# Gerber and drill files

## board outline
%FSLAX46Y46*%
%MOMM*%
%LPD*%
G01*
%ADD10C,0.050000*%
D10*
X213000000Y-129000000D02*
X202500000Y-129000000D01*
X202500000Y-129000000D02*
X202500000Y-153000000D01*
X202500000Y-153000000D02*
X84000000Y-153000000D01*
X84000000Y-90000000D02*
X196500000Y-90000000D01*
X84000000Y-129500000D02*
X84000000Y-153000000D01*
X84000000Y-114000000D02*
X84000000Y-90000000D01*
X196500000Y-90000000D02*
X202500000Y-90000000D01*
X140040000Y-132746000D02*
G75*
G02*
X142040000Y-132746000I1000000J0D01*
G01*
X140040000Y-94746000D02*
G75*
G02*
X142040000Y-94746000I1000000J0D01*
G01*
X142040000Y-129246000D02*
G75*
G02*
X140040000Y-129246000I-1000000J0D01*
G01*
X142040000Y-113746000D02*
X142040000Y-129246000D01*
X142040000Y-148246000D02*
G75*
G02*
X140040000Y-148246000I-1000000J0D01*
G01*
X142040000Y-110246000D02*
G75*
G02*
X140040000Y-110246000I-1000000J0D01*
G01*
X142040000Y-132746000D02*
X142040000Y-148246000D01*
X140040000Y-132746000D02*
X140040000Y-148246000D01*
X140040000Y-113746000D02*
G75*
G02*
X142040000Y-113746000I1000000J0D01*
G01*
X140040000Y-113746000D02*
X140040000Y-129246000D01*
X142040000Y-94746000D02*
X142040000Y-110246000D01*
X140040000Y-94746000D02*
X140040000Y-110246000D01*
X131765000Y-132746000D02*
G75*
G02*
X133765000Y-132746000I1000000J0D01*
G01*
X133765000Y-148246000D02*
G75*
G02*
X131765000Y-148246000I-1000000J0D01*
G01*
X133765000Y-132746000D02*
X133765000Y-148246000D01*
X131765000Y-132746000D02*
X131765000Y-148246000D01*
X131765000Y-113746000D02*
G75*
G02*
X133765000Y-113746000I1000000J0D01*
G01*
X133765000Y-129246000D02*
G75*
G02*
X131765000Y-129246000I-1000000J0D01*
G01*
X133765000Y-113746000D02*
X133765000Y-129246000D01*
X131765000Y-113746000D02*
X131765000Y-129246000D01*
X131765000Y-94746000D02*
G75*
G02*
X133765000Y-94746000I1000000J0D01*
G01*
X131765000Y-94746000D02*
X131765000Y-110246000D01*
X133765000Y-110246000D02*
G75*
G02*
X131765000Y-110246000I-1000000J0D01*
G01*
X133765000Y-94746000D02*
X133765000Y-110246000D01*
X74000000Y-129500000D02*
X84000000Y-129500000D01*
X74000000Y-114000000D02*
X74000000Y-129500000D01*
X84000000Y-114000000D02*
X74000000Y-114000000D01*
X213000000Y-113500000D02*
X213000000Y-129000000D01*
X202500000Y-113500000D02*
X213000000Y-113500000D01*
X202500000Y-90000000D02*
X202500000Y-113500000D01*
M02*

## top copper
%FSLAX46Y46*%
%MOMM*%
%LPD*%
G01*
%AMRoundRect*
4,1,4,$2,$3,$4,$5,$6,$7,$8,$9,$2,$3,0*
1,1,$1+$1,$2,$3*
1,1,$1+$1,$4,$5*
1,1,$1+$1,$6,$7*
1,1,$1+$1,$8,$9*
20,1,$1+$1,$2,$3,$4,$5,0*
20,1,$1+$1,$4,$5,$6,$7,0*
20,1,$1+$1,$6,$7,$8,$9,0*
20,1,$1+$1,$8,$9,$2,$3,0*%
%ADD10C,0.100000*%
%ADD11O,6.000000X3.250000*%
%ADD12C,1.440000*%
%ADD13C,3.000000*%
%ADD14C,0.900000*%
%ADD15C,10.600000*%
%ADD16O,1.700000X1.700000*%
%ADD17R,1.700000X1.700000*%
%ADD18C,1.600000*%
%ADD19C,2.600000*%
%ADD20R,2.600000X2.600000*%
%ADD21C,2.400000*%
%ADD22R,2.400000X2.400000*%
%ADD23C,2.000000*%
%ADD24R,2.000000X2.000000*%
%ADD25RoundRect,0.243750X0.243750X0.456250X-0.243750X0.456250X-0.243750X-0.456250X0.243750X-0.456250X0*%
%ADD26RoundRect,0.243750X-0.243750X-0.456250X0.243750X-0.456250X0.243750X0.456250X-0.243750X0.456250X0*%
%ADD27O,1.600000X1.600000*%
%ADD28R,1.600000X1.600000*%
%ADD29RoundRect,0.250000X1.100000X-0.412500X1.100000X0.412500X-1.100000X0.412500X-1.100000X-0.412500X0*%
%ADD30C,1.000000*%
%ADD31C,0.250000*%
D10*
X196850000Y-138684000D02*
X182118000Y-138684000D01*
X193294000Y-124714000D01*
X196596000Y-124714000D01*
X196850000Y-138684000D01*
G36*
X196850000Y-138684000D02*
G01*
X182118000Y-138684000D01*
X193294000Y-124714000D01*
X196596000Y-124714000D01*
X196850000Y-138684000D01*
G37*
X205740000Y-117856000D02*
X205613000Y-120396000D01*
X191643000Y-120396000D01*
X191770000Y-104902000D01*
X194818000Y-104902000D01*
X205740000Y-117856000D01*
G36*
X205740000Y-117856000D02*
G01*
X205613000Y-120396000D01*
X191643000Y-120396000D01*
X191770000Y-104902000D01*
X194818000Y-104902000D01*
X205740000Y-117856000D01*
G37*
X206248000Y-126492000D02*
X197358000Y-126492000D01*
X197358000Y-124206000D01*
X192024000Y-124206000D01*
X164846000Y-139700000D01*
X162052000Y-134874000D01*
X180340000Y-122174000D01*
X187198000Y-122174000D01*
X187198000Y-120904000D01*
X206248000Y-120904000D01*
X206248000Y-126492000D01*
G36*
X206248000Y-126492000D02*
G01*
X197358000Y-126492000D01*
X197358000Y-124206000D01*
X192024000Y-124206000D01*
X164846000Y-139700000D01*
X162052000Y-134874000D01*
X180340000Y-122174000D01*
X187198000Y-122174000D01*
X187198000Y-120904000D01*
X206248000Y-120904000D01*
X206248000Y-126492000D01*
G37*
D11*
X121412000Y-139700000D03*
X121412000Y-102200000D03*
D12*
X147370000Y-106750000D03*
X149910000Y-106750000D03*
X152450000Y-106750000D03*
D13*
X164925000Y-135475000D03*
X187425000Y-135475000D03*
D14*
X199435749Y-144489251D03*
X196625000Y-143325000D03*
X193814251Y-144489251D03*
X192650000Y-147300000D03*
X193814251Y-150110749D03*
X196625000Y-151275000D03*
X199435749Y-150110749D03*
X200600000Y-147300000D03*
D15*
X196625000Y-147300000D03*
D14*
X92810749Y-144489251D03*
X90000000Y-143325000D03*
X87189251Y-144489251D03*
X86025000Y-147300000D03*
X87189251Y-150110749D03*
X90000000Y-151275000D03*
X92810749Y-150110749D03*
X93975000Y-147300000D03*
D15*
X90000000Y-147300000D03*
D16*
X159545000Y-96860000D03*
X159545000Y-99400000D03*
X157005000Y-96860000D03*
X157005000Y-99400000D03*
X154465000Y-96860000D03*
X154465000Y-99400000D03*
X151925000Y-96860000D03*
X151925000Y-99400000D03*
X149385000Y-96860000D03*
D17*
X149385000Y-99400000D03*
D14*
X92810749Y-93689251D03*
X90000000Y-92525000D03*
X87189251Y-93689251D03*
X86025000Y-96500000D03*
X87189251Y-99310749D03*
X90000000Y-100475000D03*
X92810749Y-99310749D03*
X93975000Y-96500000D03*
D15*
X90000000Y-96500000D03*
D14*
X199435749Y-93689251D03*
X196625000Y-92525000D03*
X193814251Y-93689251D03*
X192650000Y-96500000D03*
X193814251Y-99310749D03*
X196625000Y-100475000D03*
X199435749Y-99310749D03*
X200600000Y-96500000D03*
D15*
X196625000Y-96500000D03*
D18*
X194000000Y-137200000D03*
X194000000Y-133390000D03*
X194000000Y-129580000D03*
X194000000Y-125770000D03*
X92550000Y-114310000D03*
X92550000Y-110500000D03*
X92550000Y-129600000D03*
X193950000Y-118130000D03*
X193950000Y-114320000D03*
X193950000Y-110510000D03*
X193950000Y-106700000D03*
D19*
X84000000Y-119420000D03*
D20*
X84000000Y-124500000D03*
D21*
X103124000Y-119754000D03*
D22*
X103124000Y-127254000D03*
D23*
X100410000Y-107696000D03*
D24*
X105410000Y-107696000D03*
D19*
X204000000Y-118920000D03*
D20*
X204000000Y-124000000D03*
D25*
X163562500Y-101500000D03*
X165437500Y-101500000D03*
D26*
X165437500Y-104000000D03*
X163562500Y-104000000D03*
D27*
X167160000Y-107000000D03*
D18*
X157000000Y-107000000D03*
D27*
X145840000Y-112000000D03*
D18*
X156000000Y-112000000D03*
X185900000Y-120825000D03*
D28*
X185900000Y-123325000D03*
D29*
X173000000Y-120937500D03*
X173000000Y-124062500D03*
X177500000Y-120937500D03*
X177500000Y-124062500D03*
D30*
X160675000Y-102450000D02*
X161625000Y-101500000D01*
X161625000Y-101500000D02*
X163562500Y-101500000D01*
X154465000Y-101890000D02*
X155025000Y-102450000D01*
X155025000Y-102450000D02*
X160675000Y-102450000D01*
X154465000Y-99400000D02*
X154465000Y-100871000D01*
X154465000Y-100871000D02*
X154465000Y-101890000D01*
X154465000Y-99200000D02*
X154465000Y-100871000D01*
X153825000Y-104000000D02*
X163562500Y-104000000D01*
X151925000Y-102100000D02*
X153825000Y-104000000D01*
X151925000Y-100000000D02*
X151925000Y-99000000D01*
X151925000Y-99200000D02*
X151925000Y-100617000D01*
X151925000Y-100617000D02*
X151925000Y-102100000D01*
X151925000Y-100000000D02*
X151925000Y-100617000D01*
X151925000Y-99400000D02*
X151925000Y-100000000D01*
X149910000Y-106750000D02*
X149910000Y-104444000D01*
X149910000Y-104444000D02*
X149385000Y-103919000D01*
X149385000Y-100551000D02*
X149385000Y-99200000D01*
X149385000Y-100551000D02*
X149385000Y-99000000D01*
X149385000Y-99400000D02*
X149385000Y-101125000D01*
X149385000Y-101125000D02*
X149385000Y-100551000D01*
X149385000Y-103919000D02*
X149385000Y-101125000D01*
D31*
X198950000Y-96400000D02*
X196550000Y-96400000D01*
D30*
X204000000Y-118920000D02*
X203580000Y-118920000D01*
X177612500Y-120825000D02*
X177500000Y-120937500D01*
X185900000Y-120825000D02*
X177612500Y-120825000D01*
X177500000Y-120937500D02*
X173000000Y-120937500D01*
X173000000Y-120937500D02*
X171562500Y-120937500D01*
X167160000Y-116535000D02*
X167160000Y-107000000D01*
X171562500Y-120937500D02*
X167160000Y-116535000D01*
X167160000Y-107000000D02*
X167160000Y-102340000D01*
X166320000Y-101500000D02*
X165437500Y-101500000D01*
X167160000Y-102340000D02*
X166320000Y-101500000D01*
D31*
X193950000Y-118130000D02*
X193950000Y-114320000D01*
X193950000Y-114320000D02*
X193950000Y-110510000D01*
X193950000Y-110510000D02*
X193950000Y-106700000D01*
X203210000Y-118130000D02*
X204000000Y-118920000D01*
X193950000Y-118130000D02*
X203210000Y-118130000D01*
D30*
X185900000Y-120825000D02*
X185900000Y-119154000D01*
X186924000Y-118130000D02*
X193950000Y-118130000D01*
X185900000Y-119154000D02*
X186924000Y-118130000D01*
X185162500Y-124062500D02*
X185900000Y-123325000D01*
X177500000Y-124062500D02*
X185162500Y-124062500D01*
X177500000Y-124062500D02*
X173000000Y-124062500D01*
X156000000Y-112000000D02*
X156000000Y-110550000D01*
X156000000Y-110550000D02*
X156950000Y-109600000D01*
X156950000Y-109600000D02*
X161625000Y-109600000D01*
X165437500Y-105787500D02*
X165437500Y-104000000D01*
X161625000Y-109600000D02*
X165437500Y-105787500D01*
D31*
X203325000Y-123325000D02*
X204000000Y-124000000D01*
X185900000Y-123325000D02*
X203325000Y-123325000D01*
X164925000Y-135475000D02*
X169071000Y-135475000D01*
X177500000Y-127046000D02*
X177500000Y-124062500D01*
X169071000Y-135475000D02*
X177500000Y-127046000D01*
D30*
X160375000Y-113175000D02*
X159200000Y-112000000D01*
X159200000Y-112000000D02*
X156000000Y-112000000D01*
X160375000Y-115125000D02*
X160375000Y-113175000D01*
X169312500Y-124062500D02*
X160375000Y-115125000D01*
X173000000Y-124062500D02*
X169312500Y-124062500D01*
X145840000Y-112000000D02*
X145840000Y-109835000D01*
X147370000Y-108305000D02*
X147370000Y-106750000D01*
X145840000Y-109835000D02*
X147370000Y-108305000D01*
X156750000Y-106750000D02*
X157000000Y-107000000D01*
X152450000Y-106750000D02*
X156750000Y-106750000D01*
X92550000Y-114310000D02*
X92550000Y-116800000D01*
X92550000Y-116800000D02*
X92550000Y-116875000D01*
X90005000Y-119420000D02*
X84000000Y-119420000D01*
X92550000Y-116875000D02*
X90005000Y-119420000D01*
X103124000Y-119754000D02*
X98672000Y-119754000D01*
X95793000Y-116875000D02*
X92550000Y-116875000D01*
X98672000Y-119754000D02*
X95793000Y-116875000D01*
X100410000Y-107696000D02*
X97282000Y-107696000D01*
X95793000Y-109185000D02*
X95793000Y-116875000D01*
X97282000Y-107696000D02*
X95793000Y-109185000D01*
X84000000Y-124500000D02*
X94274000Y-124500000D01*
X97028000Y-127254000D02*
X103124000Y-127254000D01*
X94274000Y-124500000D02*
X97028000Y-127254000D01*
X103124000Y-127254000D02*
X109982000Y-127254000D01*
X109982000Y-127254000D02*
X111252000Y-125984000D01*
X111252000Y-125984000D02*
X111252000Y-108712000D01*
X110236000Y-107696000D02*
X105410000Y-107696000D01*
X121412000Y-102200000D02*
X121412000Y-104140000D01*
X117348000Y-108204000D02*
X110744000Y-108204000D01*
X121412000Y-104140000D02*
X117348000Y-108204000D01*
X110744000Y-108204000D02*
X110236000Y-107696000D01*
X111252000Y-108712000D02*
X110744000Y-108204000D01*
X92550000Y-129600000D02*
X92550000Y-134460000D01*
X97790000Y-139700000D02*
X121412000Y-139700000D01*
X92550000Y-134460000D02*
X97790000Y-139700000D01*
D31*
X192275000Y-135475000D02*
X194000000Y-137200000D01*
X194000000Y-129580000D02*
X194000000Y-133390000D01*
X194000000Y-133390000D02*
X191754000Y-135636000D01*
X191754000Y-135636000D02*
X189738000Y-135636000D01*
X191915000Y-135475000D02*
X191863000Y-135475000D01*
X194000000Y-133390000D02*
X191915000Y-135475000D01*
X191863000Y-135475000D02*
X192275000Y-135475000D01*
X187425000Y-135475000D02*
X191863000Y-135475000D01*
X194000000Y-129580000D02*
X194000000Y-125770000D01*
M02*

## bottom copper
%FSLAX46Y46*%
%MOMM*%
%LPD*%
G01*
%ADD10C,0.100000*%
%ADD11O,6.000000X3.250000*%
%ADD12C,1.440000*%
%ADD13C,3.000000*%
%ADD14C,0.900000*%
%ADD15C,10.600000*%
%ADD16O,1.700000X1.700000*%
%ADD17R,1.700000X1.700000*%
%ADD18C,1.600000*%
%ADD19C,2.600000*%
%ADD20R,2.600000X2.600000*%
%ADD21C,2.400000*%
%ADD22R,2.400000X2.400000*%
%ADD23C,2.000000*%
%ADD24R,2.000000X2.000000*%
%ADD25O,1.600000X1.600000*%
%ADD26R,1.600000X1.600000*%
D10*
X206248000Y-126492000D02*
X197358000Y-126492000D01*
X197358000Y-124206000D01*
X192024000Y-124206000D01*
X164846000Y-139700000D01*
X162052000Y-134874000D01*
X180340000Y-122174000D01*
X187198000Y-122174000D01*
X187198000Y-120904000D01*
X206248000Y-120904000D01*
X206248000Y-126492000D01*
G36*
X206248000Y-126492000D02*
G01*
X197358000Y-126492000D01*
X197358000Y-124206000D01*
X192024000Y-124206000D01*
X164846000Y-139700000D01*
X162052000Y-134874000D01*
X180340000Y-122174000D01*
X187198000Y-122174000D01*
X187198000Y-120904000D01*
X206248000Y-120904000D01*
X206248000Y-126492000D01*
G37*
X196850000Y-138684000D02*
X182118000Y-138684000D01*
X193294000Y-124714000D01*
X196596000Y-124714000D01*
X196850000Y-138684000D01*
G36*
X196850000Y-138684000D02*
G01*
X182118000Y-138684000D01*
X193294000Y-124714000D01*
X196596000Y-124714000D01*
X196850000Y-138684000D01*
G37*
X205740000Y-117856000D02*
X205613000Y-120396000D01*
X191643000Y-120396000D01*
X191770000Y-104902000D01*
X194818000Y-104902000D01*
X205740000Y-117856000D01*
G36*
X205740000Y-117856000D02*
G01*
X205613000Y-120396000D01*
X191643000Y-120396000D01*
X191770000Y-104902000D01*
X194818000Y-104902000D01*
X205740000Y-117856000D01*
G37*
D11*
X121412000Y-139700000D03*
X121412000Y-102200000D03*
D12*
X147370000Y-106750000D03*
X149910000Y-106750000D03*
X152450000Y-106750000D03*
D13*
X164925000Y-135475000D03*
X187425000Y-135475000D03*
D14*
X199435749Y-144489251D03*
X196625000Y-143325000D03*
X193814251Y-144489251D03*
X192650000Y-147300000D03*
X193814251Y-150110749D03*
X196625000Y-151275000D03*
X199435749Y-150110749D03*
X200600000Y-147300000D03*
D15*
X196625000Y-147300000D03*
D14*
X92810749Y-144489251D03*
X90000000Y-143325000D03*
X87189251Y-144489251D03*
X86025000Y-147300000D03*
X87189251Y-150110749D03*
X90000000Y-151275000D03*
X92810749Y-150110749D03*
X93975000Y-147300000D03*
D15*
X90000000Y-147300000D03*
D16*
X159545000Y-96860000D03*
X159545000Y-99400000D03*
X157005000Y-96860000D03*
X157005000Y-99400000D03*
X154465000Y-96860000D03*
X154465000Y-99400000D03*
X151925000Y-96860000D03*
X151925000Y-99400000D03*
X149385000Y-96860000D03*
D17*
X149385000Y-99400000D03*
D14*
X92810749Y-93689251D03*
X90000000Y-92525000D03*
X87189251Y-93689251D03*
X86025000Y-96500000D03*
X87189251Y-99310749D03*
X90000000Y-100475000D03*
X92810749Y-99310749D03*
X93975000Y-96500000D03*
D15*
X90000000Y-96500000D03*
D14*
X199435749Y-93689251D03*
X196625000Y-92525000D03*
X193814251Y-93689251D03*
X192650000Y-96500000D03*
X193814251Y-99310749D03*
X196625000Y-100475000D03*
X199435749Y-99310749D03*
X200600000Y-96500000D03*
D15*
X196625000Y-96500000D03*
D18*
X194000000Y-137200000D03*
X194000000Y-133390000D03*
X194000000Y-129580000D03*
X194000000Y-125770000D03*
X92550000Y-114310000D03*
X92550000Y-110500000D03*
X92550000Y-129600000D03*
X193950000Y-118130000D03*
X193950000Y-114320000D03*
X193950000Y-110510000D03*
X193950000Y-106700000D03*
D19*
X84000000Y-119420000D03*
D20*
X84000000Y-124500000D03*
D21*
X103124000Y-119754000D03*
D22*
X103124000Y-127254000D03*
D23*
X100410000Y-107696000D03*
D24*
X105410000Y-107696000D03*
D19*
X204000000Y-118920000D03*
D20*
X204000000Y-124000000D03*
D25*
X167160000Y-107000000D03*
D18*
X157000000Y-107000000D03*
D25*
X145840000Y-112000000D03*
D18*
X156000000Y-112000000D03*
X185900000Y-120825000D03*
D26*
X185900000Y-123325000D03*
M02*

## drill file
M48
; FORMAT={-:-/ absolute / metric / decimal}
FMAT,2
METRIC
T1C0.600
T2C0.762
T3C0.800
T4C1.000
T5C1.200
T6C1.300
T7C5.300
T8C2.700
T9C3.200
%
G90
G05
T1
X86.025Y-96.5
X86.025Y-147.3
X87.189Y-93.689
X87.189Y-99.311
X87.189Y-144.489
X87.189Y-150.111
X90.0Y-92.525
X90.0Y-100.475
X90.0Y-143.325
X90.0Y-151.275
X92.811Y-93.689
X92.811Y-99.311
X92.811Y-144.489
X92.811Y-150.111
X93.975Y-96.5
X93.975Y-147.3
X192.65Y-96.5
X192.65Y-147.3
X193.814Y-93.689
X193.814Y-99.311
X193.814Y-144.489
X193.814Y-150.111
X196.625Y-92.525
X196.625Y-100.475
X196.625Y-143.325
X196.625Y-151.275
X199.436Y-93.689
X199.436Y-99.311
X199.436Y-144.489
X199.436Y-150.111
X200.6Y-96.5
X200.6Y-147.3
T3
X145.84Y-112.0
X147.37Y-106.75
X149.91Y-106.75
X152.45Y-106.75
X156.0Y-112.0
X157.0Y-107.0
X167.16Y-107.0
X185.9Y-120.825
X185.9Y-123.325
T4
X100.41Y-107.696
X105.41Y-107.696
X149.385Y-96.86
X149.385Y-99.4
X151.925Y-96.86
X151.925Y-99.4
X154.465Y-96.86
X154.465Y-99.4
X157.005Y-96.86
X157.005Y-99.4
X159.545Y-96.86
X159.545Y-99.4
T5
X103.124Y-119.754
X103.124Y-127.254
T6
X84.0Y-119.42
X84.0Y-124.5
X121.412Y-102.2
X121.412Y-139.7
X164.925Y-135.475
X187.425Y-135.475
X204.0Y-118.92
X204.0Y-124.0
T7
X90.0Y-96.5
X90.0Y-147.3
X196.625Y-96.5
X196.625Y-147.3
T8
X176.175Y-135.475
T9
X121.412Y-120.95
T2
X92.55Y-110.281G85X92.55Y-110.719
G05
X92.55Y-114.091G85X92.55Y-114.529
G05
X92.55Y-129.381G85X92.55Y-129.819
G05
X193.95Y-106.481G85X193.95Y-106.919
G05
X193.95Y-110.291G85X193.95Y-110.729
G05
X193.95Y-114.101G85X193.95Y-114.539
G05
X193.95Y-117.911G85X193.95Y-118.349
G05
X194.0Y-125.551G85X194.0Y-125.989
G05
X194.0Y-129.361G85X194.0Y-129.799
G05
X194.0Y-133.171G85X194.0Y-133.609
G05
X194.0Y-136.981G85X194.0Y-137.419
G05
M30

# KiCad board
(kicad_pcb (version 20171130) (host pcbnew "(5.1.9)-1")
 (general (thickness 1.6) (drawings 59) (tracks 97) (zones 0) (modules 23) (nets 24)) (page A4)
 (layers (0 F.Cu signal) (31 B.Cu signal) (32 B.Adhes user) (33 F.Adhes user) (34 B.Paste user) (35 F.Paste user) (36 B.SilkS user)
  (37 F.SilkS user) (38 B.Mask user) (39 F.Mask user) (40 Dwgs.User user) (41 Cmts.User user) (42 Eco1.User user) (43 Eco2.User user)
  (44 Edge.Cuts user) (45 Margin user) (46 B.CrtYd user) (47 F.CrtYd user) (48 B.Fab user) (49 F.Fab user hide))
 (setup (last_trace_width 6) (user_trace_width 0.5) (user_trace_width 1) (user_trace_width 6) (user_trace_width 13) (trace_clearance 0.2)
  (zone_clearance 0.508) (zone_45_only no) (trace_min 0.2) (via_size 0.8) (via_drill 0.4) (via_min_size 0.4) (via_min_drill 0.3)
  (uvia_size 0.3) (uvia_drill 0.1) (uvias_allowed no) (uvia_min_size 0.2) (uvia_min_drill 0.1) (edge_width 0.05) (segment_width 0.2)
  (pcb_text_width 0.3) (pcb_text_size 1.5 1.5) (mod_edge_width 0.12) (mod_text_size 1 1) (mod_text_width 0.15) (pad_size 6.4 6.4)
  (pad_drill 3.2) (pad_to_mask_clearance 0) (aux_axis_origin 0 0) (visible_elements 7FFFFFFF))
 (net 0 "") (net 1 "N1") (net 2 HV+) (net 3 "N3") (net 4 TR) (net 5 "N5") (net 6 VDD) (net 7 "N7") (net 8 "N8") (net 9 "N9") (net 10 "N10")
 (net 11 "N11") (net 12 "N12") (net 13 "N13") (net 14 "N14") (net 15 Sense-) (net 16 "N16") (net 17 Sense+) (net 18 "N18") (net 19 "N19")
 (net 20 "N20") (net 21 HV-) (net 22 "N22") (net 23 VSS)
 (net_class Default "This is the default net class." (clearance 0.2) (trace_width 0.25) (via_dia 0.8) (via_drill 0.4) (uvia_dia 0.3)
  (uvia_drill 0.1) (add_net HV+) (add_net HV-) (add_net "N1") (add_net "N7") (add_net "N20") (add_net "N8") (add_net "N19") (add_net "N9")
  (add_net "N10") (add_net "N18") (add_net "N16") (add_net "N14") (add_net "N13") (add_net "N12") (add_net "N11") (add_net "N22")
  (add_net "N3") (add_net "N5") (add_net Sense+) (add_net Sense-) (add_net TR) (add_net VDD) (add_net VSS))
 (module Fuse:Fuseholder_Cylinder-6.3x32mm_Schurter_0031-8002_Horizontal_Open (layer F.Cu) (at 121.412 139.7 90)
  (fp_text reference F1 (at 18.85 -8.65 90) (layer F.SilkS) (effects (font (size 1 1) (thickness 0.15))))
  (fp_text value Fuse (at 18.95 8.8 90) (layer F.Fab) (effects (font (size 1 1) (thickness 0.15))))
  (pad 1 thru_hole oval (at 0 0 90) (size 3.25 6) (drill 1.3) (layers *.Cu *.Mask) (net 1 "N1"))
  (pad 2 thru_hole oval (at 37.5 0 90) (size 3.25 6) (drill 1.3) (layers *.Cu *.Mask) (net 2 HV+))
  (pad "" np_thru_hole circle (at 18.75 0 90) (size 3.2 3.2) (drill 3.2) (layers *.Cu *.Mask)))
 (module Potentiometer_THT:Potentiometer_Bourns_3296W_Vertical (layer F.Cu) (at 152.45 106.75)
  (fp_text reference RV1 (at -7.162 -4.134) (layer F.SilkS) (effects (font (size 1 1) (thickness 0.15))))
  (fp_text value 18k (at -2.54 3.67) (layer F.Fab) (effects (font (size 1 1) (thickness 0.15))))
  (pad 3 thru_hole circle (at -5.08 0) (size 1.44 1.44) (drill 0.8) (layers *.Cu *.Mask) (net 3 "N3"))
  (pad 2 thru_hole circle (at -2.54 0) (size 1.44 1.44) (drill 0.8) (layers *.Cu *.Mask) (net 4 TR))
  (pad 1 thru_hole circle (at 0 0) (size 1.44 1.44) (drill 0.8) (layers *.Cu *.Mask) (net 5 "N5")))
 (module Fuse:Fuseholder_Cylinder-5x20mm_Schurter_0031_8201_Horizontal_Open (layer F.Cu) (at 187.425 135.475 180)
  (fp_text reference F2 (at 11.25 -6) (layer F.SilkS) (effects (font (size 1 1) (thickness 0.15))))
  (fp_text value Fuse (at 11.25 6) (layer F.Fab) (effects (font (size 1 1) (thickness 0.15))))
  (pad "" np_thru_hole circle (at 11.25 0 180) (size 2.7 2.7) (drill 2.7) (layers *.Cu *.Mask))
  (pad 2 thru_hole circle (at 22.5 0 180) (size 3 3) (drill 1.3) (layers *.Cu *.Mask) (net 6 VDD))
  (pad 1 thru_hole circle (at 0 0 180) (size 3 3) (drill 1.3) (layers *.Cu *.Mask) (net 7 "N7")))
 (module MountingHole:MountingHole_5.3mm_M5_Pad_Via (layer F.Cu) (at 196.625 147.3)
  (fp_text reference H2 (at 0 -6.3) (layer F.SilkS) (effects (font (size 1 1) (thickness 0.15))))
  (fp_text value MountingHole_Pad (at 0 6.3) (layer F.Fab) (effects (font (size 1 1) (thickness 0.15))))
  (pad 1 thru_hole circle (at 2.810749 -2.810749) (size 0.9 0.9) (drill 0.6) (layers *.Cu *.Mask) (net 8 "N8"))
  (pad 1 thru_hole circle (at 0 -3.975) (size 0.9 0.9) (drill 0.6) (layers *.Cu *.Mask) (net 8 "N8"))
  (pad 1 thru_hole circle (at -2.810749 -2.810749) (size 0.9 0.9) (drill 0.6) (layers *.Cu *.Mask) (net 8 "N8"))
  (pad 1 thru_hole circle (at -3.975 0) (size 0.9 0.9) (drill 0.6) (layers *.Cu *.Mask) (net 8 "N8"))
  (pad 1 thru_hole circle (at -2.810749 2.810749) (size 0.9 0.9) (drill 0.6) (layers *.Cu *.Mask) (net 8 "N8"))
  (pad 1 thru_hole circle (at 0 3.975) (size 0.9 0.9) (drill 0.6) (layers *.Cu *.Mask) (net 8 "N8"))
  (pad 1 thru_hole circle (at 2.810749 2.810749) (size 0.9 0.9) (drill 0.6) (layers *.Cu *.Mask) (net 8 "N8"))
  (pad 1 thru_hole circle (at 3.975 0) (size 0.9 0.9) (drill 0.6) (layers *.Cu *.Mask) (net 8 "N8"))
  (pad 1 thru_hole circle (at 0 0) (size 10.6 10.6) (drill 5.3) (layers *.Cu *.Mask) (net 8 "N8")))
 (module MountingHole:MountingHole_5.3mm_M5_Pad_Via (layer F.Cu) (at 90 147.3)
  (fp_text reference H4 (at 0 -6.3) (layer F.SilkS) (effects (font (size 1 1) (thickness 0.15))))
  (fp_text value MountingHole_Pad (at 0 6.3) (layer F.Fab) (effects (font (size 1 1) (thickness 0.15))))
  (pad 1 thru_hole circle (at 2.810749 -2.810749) (size 0.9 0.9) (drill 0.6) (layers *.Cu *.Mask) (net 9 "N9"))
  (pad 1 thru_hole circle (at 0 -3.975) (size 0.9 0.9) (drill 0.6) (layers *.Cu *.Mask) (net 9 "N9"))
  (pad 1 thru_hole circle (at -2.810749 -2.810749) (size 0.9 0.9) (drill 0.6) (layers *.Cu *.Mask) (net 9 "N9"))
  (pad 1 thru_hole circle (at -3.975 0) (size 0.9 0.9) (drill 0.6) (layers *.Cu *.Mask) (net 9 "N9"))
  (pad 1 thru_hole circle (at -2.810749 2.810749) (size 0.9 0.9) (drill 0.6) (layers *.Cu *.Mask) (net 9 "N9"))
  (pad 1 thru_hole circle (at 0 3.975) (size 0.9 0.9) (drill 0.6) (layers *.Cu *.Mask) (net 9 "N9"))
  (pad 1 thru_hole circle (at 2.810749 2.810749) (size 0.9 0.9) (drill 0.6) (layers *.Cu *.Mask) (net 9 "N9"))
  (pad 1 thru_hole circle (at 3.975 0) (size 0.9 0.9) (drill 0.6) (layers *.Cu *.Mask) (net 9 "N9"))
  (pad 1 thru_hole circle (at 0 0) (size 10.6 10.6) (drill 5.3) (layers *.Cu *.Mask) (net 9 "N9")))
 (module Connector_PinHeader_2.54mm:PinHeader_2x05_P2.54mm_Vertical (layer F.Cu) (at 149.385 99.4 90)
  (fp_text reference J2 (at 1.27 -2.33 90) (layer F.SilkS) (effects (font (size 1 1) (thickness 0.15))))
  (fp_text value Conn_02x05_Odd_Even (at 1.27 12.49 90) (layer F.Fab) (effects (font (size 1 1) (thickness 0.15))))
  (pad 10 thru_hole oval (at 2.54 10.16 90) (size 1.7 1.7) (drill 1) (layers *.Cu *.Mask) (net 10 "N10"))
  (pad 9 thru_hole oval (at 0 10.16 90) (size 1.7 1.7) (drill 1) (layers *.Cu *.Mask) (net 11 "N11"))
  (pad 8 thru_hole oval (at 2.54 7.62 90) (size 1.7 1.7) (drill 1) (layers *.Cu *.Mask) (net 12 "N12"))
  (pad 7 thru_hole oval (at 0 7.62 90) (size 1.7 1.7) (drill 1) (layers *.Cu *.Mask) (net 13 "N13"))
  (pad 6 thru_hole oval (at 2.54 5.08 90) (size 1.7 1.7) (drill 1) (layers *.Cu *.Mask) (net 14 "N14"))
  (pad 5 thru_hole oval (at 0 5.08 90) (size 1.7 1.7) (drill 1) (layers *.Cu *.Mask) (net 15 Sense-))
  (pad 4 thru_hole oval (at 2.54 2.54 90) (size 1.7 1.7) (drill 1) (layers *.Cu *.Mask) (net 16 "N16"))
  (pad 3 thru_hole oval (at 0 2.54 90) (size 1.7 1.7) (drill 1) (layers *.Cu *.Mask) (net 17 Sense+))
  (pad 2 thru_hole oval (at 2.54 0 90) (size 1.7 1.7) (drill 1) (layers *.Cu *.Mask) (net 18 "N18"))
  (pad 1 thru_hole rect (at 0 0 90) (size 1.7 1.7) (drill 1) (layers *.Cu *.Mask) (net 4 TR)))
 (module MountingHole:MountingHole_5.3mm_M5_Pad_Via (layer F.Cu) (at 90 96.5)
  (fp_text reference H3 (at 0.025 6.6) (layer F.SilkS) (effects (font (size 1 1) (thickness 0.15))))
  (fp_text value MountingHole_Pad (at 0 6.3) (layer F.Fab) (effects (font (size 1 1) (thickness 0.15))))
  (pad 1 thru_hole circle (at 2.810749 -2.810749) (size 0.9 0.9) (drill 0.6) (layers *.Cu *.Mask) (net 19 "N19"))
  (pad 1 thru_hole circle (at 0 -3.975) (size 0.9 0.9) (drill 0.6) (layers *.Cu *.Mask) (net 19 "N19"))
  (pad 1 thru_hole circle (at -2.810749 -2.810749) (size 0.9 0.9) (drill 0.6) (layers *.Cu *.Mask) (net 19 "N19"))
  (pad 1 thru_hole circle (at -3.975 0) (size 0.9 0.9) (drill 0.6) (layers *.Cu *.Mask) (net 19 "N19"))
  (pad 1 thru_hole circle (at -2.810749 2.810749) (size 0.9 0.9) (drill 0.6) (layers *.Cu *.Mask) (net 19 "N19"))
  (pad 1 thru_hole circle (at 0 3.975) (size 0.9 0.9) (drill 0.6) (layers *.Cu *.Mask) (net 19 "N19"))
  (pad 1 thru_hole circle (at 2.810749 2.810749) (size 0.9 0.9) (drill 0.6) (layers *.Cu *.Mask) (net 19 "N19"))
  (pad 1 thru_hole circle (at 3.975 0) (size 0.9 0.9) (drill 0.6) (layers *.Cu *.Mask) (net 19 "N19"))
  (pad 1 thru_hole circle (at 0 0) (size 10.6 10.6) (drill 5.3) (layers *.Cu *.Mask) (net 19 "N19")))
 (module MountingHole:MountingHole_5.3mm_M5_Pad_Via (layer F.Cu) (at 196.625 96.5)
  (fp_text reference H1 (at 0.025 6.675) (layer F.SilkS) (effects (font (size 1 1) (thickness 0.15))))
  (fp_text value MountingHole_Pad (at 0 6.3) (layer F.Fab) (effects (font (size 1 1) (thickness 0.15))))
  (pad 1 thru_hole circle (at 2.810749 -2.810749) (size 0.9 0.9) (drill 0.6) (layers *.Cu *.Mask) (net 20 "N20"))
  (pad 1 thru_hole circle (at 0 -3.975) (size 0.9 0.9) (drill 0.6) (layers *.Cu *.Mask) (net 20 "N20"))
  (pad 1 thru_hole circle (at -2.810749 -2.810749) (size 0.9 0.9) (drill 0.6) (layers *.Cu *.Mask) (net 20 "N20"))
  (pad 1 thru_hole circle (at -3.975 0) (size 0.9 0.9) (drill 0.6) (layers *.Cu *.Mask) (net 20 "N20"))
  (pad 1 thru_hole circle (at -2.810749 2.810749) (size 0.9 0.9) (drill 0.6) (layers *.Cu *.Mask) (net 20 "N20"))
  (pad 1 thru_hole circle (at 0 3.975) (size 0.9 0.9) (drill 0.6) (layers *.Cu *.Mask) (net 20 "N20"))
  (pad 1 thru_hole circle (at 2.810749 2.810749) (size 0.9 0.9) (drill 0.6) (layers *.Cu *.Mask) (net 20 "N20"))
  (pad 1 thru_hole circle (at 3.975 0) (size 0.9 0.9) (drill 0.6) (layers *.Cu *.Mask) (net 20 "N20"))
  (pad 1 thru_hole circle (at 0 0) (size 10.6 10.6) (drill 5.3) (layers *.Cu *.Mask) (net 20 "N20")))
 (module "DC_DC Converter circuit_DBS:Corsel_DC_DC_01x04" (layer F.Cu) (at 194 130.85)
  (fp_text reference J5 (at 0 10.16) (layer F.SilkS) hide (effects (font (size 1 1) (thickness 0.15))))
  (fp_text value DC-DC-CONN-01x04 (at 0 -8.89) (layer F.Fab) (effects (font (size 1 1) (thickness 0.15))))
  (pad 4 thru_hole circle (at 0 6.35) (size 1.6 1.6) (drill oval 0.762 1.2) (layers *.Cu *.Mask) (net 7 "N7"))
  (pad 3 thru_hole circle (at 0 2.54) (size 1.6 1.6) (drill oval 0.762 1.2) (layers *.Cu *.Mask) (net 7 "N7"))
  (pad 2 thru_hole circle (at 0 -1.27) (size 1.6 1.6) (drill oval 0.762 1.2) (layers *.Cu *.Mask) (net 7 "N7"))
  (pad 1 thru_hole circle (at 0 -5.08) (size 1.6 1.6) (drill oval 0.762 1.2) (layers *.Cu *.Mask) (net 7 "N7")))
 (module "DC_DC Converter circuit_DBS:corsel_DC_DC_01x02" (layer F.Cu) (at 92.55 111.5)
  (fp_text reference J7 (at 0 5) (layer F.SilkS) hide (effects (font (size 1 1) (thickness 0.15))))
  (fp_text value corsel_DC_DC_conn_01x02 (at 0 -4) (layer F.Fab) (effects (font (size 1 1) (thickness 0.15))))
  (pad 2 thru_hole circle (at 0 2.81) (size 1.6 1.6) (drill oval 0.762 1.2) (layers *.Cu *.Mask) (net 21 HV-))
  (pad 1 thru_hole circle (at 0 -1) (size 1.6 1.6) (drill oval 0.762 1.2) (layers *.Cu *.Mask) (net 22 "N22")))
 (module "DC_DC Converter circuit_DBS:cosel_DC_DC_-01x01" (layer F.Cu) (at 92.55 129.6)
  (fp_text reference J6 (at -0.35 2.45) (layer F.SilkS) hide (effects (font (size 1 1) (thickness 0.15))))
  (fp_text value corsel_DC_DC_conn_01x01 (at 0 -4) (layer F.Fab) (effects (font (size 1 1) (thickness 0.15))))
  (pad 1 thru_hole circle (at 0 0) (size 1.6 1.6) (drill oval 0.762 1.2) (layers *.Cu *.Mask) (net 1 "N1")))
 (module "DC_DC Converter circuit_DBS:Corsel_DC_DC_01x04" (layer F.Cu) (at 193.95 111.78)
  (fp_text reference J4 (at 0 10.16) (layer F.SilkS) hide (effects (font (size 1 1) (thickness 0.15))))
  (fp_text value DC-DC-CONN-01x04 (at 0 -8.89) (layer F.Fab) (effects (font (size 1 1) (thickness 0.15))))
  (pad 4 thru_hole circle (at 0 6.35) (size 1.6 1.6) (drill oval 0.762 1.2) (layers *.Cu *.Mask) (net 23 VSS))
  (pad 3 thru_hole circle (at 0 2.54) (size 1.6 1.6) (drill oval 0.762 1.2) (layers *.Cu *.Mask) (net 23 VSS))
  (pad 2 thru_hole circle (at 0 -1.27) (size 1.6 1.6) (drill oval 0.762 1.2) (layers *.Cu *.Mask) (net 23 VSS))
  (pad 1 thru_hole circle (at 0 -5.08) (size 1.6 1.6) (drill oval 0.762 1.2) (layers *.Cu *.Mask) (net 23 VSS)))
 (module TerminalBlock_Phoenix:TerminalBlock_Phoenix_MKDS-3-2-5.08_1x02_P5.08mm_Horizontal (layer F.Cu) (at 84 124.5 90)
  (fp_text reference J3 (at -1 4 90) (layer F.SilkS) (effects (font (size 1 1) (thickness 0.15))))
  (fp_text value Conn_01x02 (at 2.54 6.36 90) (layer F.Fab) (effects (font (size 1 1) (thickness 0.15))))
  (pad 2 thru_hole circle (at 5.08 0 90) (size 2.6 2.6) (drill 1.3) (layers *.Cu *.Mask) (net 21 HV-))
  (pad 1 thru_hole rect (at 0 0 90) (size 2.6 2.6) (drill 1.3) (layers *.Cu *.Mask) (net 2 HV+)))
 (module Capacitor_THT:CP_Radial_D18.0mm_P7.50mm (layer F.Cu) (at 103.124 127.254 90)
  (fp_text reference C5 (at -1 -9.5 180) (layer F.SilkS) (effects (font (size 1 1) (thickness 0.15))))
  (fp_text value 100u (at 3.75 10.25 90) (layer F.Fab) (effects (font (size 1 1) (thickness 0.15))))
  (pad 2 thru_hole circle (at 7.5 0 90) (size 2.4 2.4) (drill 1.2) (layers *.Cu *.Mask) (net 21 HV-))
  (pad 1 thru_hole rect (at 0 0 90) (size 2.4 2.4) (drill 1.2) (layers *.Cu *.Mask) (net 2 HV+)))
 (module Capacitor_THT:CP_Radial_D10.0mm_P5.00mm (layer F.Cu) (at 105.41 107.696 180)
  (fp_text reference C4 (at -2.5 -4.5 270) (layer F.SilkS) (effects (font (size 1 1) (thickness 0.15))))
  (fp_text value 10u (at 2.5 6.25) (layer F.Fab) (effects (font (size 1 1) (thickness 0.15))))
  (pad 2 thru_hole circle (at 5 0 180) (size 2 2) (drill 1) (layers *.Cu *.Mask) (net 21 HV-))
  (pad 1 thru_hole rect (at 0 0 180) (size 2 2) (drill 1) (layers *.Cu *.Mask) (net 2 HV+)))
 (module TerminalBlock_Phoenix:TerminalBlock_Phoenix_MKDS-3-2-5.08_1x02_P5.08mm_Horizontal (layer F.Cu) (at 204 124 90)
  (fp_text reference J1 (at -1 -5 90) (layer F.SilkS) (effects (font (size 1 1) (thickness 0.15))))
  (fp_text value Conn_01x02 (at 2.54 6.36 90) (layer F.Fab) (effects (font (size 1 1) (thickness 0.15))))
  (pad 2 thru_hole circle (at 5.08 0 90) (size 2.6 2.6) (drill 1.3) (layers *.Cu *.Mask) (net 23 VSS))
  (pad 1 thru_hole rect (at 0 0 90) (size 2.6 2.6) (drill 1.3) (layers *.Cu *.Mask) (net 6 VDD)))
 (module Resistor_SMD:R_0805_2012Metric (layer F.Cu) (at 164.5 101.5 180)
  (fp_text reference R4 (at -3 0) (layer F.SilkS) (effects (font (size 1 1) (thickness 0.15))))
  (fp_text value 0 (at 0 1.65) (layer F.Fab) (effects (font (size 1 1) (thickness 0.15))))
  (pad 2 smd roundrect (at 0.9375 0 180) (size 0.975 1.4) (layers F.Cu F.Paste F.Mask) (roundrect_rratio 0.25) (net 15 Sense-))
  (pad 1 smd roundrect (at -0.9375 0 180) (size 0.975 1.4) (layers F.Cu F.Paste F.Mask) (roundrect_rratio 0.25) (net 23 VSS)))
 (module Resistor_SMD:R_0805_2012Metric (layer F.Cu) (at 164.5 104)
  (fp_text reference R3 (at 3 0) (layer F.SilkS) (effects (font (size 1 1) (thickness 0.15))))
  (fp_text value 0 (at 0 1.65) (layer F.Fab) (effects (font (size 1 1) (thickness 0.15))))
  (pad 2 smd roundrect (at 0.9375 0) (size 0.975 1.4) (layers F.Cu F.Paste F.Mask) (roundrect_rratio 0.25) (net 6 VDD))
  (pad 1 smd roundrect (at -0.9375 0) (size 0.975 1.4) (layers F.Cu F.Paste F.Mask) (roundrect_rratio 0.25) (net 17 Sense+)))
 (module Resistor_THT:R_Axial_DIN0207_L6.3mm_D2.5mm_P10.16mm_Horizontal (layer F.Cu) (at 157 107)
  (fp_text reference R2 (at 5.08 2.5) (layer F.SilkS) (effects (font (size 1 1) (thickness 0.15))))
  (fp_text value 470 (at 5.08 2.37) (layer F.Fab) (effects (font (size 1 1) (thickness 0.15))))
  (pad 2 thru_hole oval (at 10.16 0) (size 1.6 1.6) (drill 0.8) (layers *.Cu *.Mask) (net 23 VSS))
  (pad 1 thru_hole circle (at 0 0) (size 1.6 1.6) (drill 0.8) (layers *.Cu *.Mask) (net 5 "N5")))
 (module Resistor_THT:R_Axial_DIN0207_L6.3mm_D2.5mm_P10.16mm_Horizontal (layer F.Cu) (at 156 112 180)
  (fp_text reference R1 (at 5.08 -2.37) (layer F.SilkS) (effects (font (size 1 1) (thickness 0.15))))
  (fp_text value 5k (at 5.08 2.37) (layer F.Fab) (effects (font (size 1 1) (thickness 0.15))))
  (pad 2 thru_hole oval (at 10.16 0 180) (size 1.6 1.6) (drill 0.8) (layers *.Cu *.Mask) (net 3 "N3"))
  (pad 1 thru_hole circle (at 0 0 180) (size 1.6 1.6) (drill 0.8) (layers *.Cu *.Mask) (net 6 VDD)))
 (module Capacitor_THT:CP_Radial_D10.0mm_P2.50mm (layer F.Cu) (at 185.9 123.325 90)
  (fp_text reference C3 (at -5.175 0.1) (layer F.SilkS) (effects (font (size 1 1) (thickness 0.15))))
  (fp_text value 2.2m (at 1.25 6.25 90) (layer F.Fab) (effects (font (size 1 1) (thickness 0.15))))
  (pad 2 thru_hole circle (at 2.5 0 90) (size 1.6 1.6) (drill 0.8) (layers *.Cu *.Mask) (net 23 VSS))
  (pad 1 thru_hole rect (at 0 0 90) (size 1.6 1.6) (drill 0.8) (layers *.Cu *.Mask) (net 6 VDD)))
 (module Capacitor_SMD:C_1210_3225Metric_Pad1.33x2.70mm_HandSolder (layer F.Cu) (at 173 122.5 90)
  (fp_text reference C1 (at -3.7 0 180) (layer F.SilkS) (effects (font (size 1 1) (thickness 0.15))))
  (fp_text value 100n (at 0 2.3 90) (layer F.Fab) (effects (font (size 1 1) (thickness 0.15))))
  (pad 2 smd roundrect (at 1.5625 0 90) (size 1.325 2.7) (layers F.Cu F.Paste F.Mask) (roundrect_rratio 0.188679) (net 23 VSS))
  (pad 1 smd roundrect (at -1.5625 0 90) (size 1.325 2.7) (layers F.Cu F.Paste F.Mask) (roundrect_rratio 0.188679) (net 6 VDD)))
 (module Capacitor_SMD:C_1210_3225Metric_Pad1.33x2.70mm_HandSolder (layer F.Cu) (at 177.5 122.5 90)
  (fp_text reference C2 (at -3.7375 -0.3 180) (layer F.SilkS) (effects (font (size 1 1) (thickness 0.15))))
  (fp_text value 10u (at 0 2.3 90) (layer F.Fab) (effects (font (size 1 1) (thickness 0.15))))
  (pad 2 smd roundrect (at 1.5625 0 90) (size 1.325 2.7) (layers F.Cu F.Paste F.Mask) (roundrect_rratio 0.188679) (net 23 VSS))
  (pad 1 smd roundrect (at -1.5625 0 90) (size 1.325 2.7) (layers F.Cu F.Paste F.Mask) (roundrect_rratio 0.188679) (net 6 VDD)))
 (gr_poly (pts (xy 196.85 138.684) (xy 182.118 138.684) (xy 193.294 124.714) (xy 196.596 124.714)) (layer F.Cu) (width 0.1))
 (gr_poly
  (pts (xy 205.74 117.856) (xy 205.613 120.396) (xy 191.643 120.396) (xy 191.77 104.902) (xy 194.818 104.902)) (layer F.Cu) (width 0.1))
 (gr_poly
  (pts (xy 206.248 126.492) (xy 197.358 126.492) (xy 197.358 124.206) (xy 192.024 124.206) (xy 164.846 139.7) (xy 162.052 134.874)
   (xy 180.34 122.174) (xy 187.198 122.174) (xy 187.198 120.904) (xy 206.248 120.904))
  (layer F.Cu) (width 0.1))
 (gr_poly
  (pts (xy 206.248 126.492) (xy 197.358 126.492) (xy 197.358 124.206) (xy 192.024 124.206) (xy 164.846 139.7) (xy 162.052 134.874)
   (xy 180.34 122.174) (xy 187.198 122.174) (xy 187.198 120.904) (xy 206.248 120.904))
  (layer B.Cu) (width 0.1))
 (gr_poly (pts (xy 196.85 138.684) (xy 182.118 138.684) (xy 193.294 124.714) (xy 196.596 124.714)) (layer B.Cu) (width 0.1))
 (gr_poly
  (pts (xy 205.74 117.856) (xy 205.613 120.396) (xy 191.643 120.396) (xy 191.77 104.902) (xy 194.818 104.902)) (layer B.Cu) (width 0.1))
 (gr_line (start 213 129) (end 202.5 129) (layer Edge.Cuts) (width 0.05))
 (gr_line (start 202.5 129) (end 202.5 153) (layer Edge.Cuts) (width 0.05))
 (gr_line (start 202.5 153) (end 84 153) (layer Edge.Cuts) (width 0.05))
 (gr_line (start 84 90) (end 196.5 90) (layer Edge.Cuts) (width 0.05))
 (gr_line (start 84 129.5) (end 84 153) (layer Edge.Cuts) (width 0.05))
 (gr_line (start 84 114) (end 84 90) (layer Edge.Cuts) (width 0.05))
 (gr_line (start 196.5 90) (end 202.5 90) (layer Edge.Cuts) (width 0.05))
 (gr_arc (start 141.04 132.746) (end 142.04 132.746) (angle -180) (layer Edge.Cuts) (width 0.05))
 (gr_arc (start 141.04 94.746) (end 142.04 94.746) (angle -180) (layer Edge.Cuts) (width 0.05))
 (gr_arc (start 141.04 129.246) (end 140.04 129.246) (angle -180) (layer Edge.Cuts) (width 0.05))
 (gr_line (start 142.04 113.746) (end 142.04 129.246) (layer Edge.Cuts) (width 0.05))
 (gr_arc (start 141.04 148.246) (end 140.04 148.246) (angle -180) (layer Edge.Cuts) (width 0.05))
 (gr_arc (start 141.04 110.246) (end 140.04 110.246) (angle -180) (layer Edge.Cuts) (width 0.05))
 (gr_line (start 142.04 132.746) (end 142.04 148.246) (layer Edge.Cuts) (width 0.05))
 (gr_line (start 140.04 132.746) (end 140.04 148.246) (layer Edge.Cuts) (width 0.05))
 (gr_arc (start 141.04 113.746) (end 142.04 113.746) (angle -180) (layer Edge.Cuts) (width 0.05))
 (gr_line (start 140.04 113.746) (end 140.04 129.246) (layer Edge.Cuts) (width 0.05))
 (gr_line (start 142.04 94.746) (end 142.04 110.246) (layer Edge.Cuts) (width 0.05))
 (gr_line (start 140.04 94.746) (end 140.04 110.246) (layer Edge.Cuts) (width 0.05))
 (gr_arc (start 132.765 132.746) (end 133.765 132.746) (angle -180) (layer Edge.Cuts) (width 0.05))
 (gr_arc (start 132.765 148.246) (end 131.765 148.246) (angle -180) (layer Edge.Cuts) (width 0.05))
 (gr_line (start 133.765 132.746) (end 133.765 148.246) (layer Edge.Cuts) (width 0.05))
 (gr_line (start 131.765 132.746) (end 131.765 148.246) (layer Edge.Cuts) (width 0.05))
 (gr_arc (start 132.765 113.746) (end 133.765 113.746) (angle -180) (layer Edge.Cuts) (width 0.05))
 (gr_arc (start 132.765 129.246) (end 131.765 129.246) (angle -180) (layer Edge.Cuts) (width 0.05))
 (gr_line (start 133.765 113.746) (end 133.765 129.246) (layer Edge.Cuts) (width 0.05))
 (gr_line (start 131.765 113.746) (end 131.765 129.246) (layer Edge.Cuts) (width 0.05))
 (gr_arc (start 132.765 94.746) (end 133.765 94.746) (angle -180) (layer Edge.Cuts) (width 0.05))
 (gr_line (start 131.765 94.746) (end 131.765 110.246) (layer Edge.Cuts) (width 0.05))
 (gr_arc (start 132.765 110.246) (end 131.765 110.246) (angle -180) (layer Edge.Cuts) (width 0.05))
 (gr_line (start 133.765 94.746) (end 133.765 110.246) (layer Edge.Cuts) (width 0.05))
 (gr_line (start 74 129.5) (end 84 129.5) (layer Edge.Cuts) (width 0.05))
 (gr_line (start 74 114) (end 74 129.5) (layer Edge.Cuts) (width 0.05))
 (gr_line (start 84 114) (end 74 114) (layer Edge.Cuts) (width 0.05))
 (gr_line (start 213 113.5) (end 213 129) (layer Edge.Cuts) (width 0.05))
 (gr_line (start 202.5 113.5) (end 213 113.5) (layer Edge.Cuts) (width 0.05))
 (gr_line (start 202.5 90) (end 202.5 113.5) (layer Edge.Cuts) (width 0.05))
 (segment (start 160.675 102.45) (end 161.625 101.5) (width 1) (layer F.Cu) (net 15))
 (segment (start 161.625 101.5) (end 163.5625 101.5) (width 1) (layer F.Cu) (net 15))
 (segment (start 154.465 101.89) (end 155.025 102.45) (width 1) (layer F.Cu) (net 15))
 (segment (start 155.025 102.45) (end 160.675 102.45) (width 1) (layer F.Cu) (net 15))
 (segment (start 154.465 99.4) (end 154.465 100.871) (width 1) (layer F.Cu) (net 15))
 (segment (start 154.465 100.871) (end 154.465 101.89) (width 1) (layer F.Cu) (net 15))
 (segment (start 154.465 99.2) (end 154.465 100.871) (width 1) (layer F.Cu) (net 15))
 (segment (start 153.825 104) (end 163.5625 104) (width 1) (layer F.Cu) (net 17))
 (segment (start 151.925 102.1) (end 153.825 104) (width 1) (layer F.Cu) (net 17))
 (segment (start 151.925 100) (end 151.925 99) (width 1) (layer F.Cu) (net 17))
 (segment (start 151.925 99.2) (end 151.925 100.617) (width 1) (layer F.Cu) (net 17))
 (segment (start 151.925 100.617) (end 151.925 102.1) (width 1) (layer F.Cu) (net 17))
 (segment (start 151.925 100) (end 151.925 100.617) (width 1) (layer F.Cu) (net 17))
 (segment (start 151.925 99.4) (end 151.925 100) (width 1) (layer F.Cu) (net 17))
 (segment (start 149.91 106.75) (end 149.91 104.444) (width 1) (layer F.Cu) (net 4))
 (segment (start 149.91 104.444) (end 149.385 103.919) (width 1) (layer F.Cu) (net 4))
 (segment (start 149.385 100.551) (end 149.385 99.2) (width 1) (layer F.Cu) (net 4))
 (segment (start 149.385 100.551) (end 149.385 99) (width 1) (layer F.Cu) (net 4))
 (segment (start 149.385 99.4) (end 149.385 101.125) (width 1) (layer F.Cu) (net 4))
 (segment (start 149.385 101.125) (end 149.385 100.551) (width 1) (layer F.Cu) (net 4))
 (segment (start 149.385 103.919) (end 149.385 101.125) (width 1) (layer F.Cu) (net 4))
 (segment (start 198.95 96.4) (end 196.55 96.4) (width 0.25) (layer F.Cu) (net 20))
 (segment (start 204 118.92) (end 203.58 118.92) (width 1) (layer F.Cu) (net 23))
 (segment (start 177.6125 120.825) (end 177.5 120.9375) (width 1) (layer F.Cu) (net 23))
 (segment (start 185.9 120.825) (end 177.6125 120.825) (width 1) (layer F.Cu) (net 23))
 (segment (start 177.5 120.9375) (end 173 120.9375) (width 1) (layer F.Cu) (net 23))
 (segment (start 173 120.9375) (end 171.5625 120.9375) (width 1) (layer F.Cu) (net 23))
 (segment (start 167.16 116.535) (end 167.16 107) (width 1) (layer F.Cu) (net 23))
 (segment (start 171.5625 120.9375) (end 167.16 116.535) (width 1) (layer F.Cu) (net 23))
 (segment (start 167.16 107) (end 167.16 102.34) (width 1) (layer F.Cu) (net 23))
 (segment (start 166.32 101.5) (end 165.4375 101.5) (width 1) (layer F.Cu) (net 23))
 (segment (start 167.16 102.34) (end 166.32 101.5) (width 1) (layer F.Cu) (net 23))
 (segment (start 193.95 118.13) (end 193.95 114.32) (width 0.25) (layer F.Cu) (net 23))
 (segment (start 193.95 114.32) (end 193.95 110.51) (width 0.25) (layer F.Cu) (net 23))
 (segment (start 193.95 110.51) (end 193.95 106.7) (width 0.25) (layer F.Cu) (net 23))
 (segment (start 203.21 118.13) (end 204 118.92) (width 0.25) (layer F.Cu) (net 23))
 (segment (start 193.95 118.13) (end 203.21 118.13) (width 0.25) (layer F.Cu) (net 23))
 (segment (start 185.9 120.825) (end 185.9 119.154) (width 1) (layer F.Cu) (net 23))
 (segment (start 186.924 118.13) (end 193.95 118.13) (width 1) (layer F.Cu) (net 23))
 (segment (start 185.9 119.154) (end 186.924 118.13) (width 1) (layer F.Cu) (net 23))
 (segment (start 185.1625 124.0625) (end 185.9 123.325) (width 1) (layer F.Cu) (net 6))
 (segment (start 177.5 124.0625) (end 185.1625 124.0625) (width 1) (layer F.Cu) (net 6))
 (segment (start 177.5 124.0625) (end 173 124.0625) (width 1) (layer F.Cu) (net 6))
 (segment (start 156 112) (end 156 110.55) (width 1) (layer F.Cu) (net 6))
 (segment (start 156 110.55) (end 156.95 109.6) (width 1) (layer F.Cu) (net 6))
 (segment (start 156.95 109.6) (end 161.625 109.6) (width 1) (layer F.Cu) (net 6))
 (segment (start 165.4375 105.7875) (end 165.4375 104) (width 1) (layer F.Cu) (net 6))
 (segment (start 161.625 109.6) (end 165.4375 105.7875) (width 1) (layer F.Cu) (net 6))
 (segment (start 203.325 123.325) (end 204 124) (width 0.25) (layer F.Cu) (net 6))
 (segment (start 185.9 123.325) (end 203.325 123.325) (width 0.25) (layer F.Cu) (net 6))
 (segment (start 164.925 135.475) (end 169.071 135.475) (width 0.25) (layer F.Cu) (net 6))
 (segment (start 177.5 127.046) (end 177.5 124.0625) (width 0.25) (layer F.Cu) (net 6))
 (segment (start 169.071 135.475) (end 177.5 127.046) (width 0.25) (layer F.Cu) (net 6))
 (segment (start 160.375 113.175) (end 159.2 112) (width 1) (layer F.Cu) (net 6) (status 1000000))
 (segment (start 159.2 112) (end 156 112) (width 1) (layer F.Cu) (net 6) (status 1000000))
 (segment (start 160.375 115.125) (end 160.375 113.175) (width 1) (layer F.Cu) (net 6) (status 1000000))
 (segment (start 169.3125 124.0625) (end 160.375 115.125) (width 1) (layer F.Cu) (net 6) (status 1000000))
 (segment (start 173 124.0625) (end 169.3125 124.0625) (width 1) (layer F.Cu) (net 6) (status 1000000))
 (segment (start 145.84 112) (end 145.84 109.835) (width 1) (layer F.Cu) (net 3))
 (segment (start 147.37 108.305) (end 147.37 106.75) (width 1) (layer F.Cu) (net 3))
 (segment (start 145.84 109.835) (end 147.37 108.305) (width 1) (layer F.Cu) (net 3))
 (segment (start 156.75 106.75) (end 157 107) (width 1) (layer F.Cu) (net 5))
 (segment (start 152.45 106.75) (end 156.75 106.75) (width 1) (layer F.Cu) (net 5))
 (segment (start 92.55 114.31) (end 92.55 116.8) (width 1) (layer F.Cu) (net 21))
 (segment (start 92.55 116.8) (end 92.55 116.875) (width 1) (layer F.Cu) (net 21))
 (segment (start 90.005 119.42) (end 84 119.42) (width 1) (layer F.Cu) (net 21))
 (segment (start 92.55 116.875) (end 90.005 119.42) (width 1) (layer F.Cu) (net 21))
 (segment (start 103.124 119.754) (end 98.672 119.754) (width 1) (layer F.Cu) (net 21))
 (segment (start 95.793 116.875) (end 92.55 116.875) (width 1) (layer F.Cu) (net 21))
 (segment (start 98.672 119.754) (end 95.793 116.875) (width 1) (layer F.Cu) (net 21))
 (segment (start 100.41 107.696) (end 97.282 107.696) (width 1) (layer F.Cu) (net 21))
 (segment (start 95.793 109.185) (end 95.793 116.875) (width 1) (layer F.Cu) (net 21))
 (segment (start 97.282 107.696) (end 95.793 109.185) (width 1) (layer F.Cu) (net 21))
 (segment (start 84 124.5) (end 94.274 124.5) (width 1) (layer F.Cu) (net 2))
 (segment (start 97.028 127.254) (end 103.124 127.254) (width 1) (layer F.Cu) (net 2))
 (segment (start 94.274 124.5) (end 97.028 127.254) (width 1) (layer F.Cu) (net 2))
 (segment (start 103.124 127.254) (end 109.982 127.254) (width 1) (layer F.Cu) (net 2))
 (segment (start 109.982 127.254) (end 111.252 125.984) (width 1) (layer F.Cu) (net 2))
 (segment (start 111.252 125.984) (end 111.252 108.712) (width 1) (layer F.Cu) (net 2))
 (segment (start 110.236 107.696) (end 105.41 107.696) (width 1) (layer F.Cu) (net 2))
 (segment (start 121.412 102.2) (end 121.412 104.14) (width 1) (layer F.Cu) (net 2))
 (segment (start 117.348 108.204) (end 110.744 108.204) (width 1) (layer F.Cu) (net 2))
 (segment (start 121.412 104.14) (end 117.348 108.204) (width 1) (layer F.Cu) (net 2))
 (segment (start 110.744 108.204) (end 110.236 107.696) (width 1) (layer F.Cu) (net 2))
 (segment (start 111.252 108.712) (end 110.744 108.204) (width 1) (layer F.Cu) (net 2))
 (segment (start 92.55 129.6) (end 92.55 134.46) (width 1) (layer F.Cu) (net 1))
 (segment (start 97.79 139.7) (end 121.412 139.7) (width 1) (layer F.Cu) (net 1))
 (segment (start 92.55 134.46) (end 97.79 139.7) (width 1) (layer F.Cu) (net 1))
 (segment (start 192.275 135.475) (end 194 137.2) (width 0.25) (layer F.Cu) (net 7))
 (segment (start 194 129.58) (end 194 133.39) (width 0.25) (layer F.Cu) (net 7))
 (segment (start 194 133.39) (end 191.754 135.636) (width 0.25) (layer F.Cu) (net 7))
 (segment (start 191.754 135.636) (end 189.738 135.636) (width 0.25) (layer F.Cu) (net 7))
 (segment (start 191.915 135.475) (end 191.863 135.475) (width 0.25) (layer F.Cu) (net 7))
 (segment (start 194 133.39) (end 191.915 135.475) (width 0.25) (layer F.Cu) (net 7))
 (segment (start 191.863 135.475) (end 192.275 135.475) (width 0.25) (layer F.Cu) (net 7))
 (segment (start 187.425 135.475) (end 191.863 135.475) (width 0.25) (layer F.Cu) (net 7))
 (segment (start 194 129.58) (end 194 125.77) (width 0.25) (layer F.Cu) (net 7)))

